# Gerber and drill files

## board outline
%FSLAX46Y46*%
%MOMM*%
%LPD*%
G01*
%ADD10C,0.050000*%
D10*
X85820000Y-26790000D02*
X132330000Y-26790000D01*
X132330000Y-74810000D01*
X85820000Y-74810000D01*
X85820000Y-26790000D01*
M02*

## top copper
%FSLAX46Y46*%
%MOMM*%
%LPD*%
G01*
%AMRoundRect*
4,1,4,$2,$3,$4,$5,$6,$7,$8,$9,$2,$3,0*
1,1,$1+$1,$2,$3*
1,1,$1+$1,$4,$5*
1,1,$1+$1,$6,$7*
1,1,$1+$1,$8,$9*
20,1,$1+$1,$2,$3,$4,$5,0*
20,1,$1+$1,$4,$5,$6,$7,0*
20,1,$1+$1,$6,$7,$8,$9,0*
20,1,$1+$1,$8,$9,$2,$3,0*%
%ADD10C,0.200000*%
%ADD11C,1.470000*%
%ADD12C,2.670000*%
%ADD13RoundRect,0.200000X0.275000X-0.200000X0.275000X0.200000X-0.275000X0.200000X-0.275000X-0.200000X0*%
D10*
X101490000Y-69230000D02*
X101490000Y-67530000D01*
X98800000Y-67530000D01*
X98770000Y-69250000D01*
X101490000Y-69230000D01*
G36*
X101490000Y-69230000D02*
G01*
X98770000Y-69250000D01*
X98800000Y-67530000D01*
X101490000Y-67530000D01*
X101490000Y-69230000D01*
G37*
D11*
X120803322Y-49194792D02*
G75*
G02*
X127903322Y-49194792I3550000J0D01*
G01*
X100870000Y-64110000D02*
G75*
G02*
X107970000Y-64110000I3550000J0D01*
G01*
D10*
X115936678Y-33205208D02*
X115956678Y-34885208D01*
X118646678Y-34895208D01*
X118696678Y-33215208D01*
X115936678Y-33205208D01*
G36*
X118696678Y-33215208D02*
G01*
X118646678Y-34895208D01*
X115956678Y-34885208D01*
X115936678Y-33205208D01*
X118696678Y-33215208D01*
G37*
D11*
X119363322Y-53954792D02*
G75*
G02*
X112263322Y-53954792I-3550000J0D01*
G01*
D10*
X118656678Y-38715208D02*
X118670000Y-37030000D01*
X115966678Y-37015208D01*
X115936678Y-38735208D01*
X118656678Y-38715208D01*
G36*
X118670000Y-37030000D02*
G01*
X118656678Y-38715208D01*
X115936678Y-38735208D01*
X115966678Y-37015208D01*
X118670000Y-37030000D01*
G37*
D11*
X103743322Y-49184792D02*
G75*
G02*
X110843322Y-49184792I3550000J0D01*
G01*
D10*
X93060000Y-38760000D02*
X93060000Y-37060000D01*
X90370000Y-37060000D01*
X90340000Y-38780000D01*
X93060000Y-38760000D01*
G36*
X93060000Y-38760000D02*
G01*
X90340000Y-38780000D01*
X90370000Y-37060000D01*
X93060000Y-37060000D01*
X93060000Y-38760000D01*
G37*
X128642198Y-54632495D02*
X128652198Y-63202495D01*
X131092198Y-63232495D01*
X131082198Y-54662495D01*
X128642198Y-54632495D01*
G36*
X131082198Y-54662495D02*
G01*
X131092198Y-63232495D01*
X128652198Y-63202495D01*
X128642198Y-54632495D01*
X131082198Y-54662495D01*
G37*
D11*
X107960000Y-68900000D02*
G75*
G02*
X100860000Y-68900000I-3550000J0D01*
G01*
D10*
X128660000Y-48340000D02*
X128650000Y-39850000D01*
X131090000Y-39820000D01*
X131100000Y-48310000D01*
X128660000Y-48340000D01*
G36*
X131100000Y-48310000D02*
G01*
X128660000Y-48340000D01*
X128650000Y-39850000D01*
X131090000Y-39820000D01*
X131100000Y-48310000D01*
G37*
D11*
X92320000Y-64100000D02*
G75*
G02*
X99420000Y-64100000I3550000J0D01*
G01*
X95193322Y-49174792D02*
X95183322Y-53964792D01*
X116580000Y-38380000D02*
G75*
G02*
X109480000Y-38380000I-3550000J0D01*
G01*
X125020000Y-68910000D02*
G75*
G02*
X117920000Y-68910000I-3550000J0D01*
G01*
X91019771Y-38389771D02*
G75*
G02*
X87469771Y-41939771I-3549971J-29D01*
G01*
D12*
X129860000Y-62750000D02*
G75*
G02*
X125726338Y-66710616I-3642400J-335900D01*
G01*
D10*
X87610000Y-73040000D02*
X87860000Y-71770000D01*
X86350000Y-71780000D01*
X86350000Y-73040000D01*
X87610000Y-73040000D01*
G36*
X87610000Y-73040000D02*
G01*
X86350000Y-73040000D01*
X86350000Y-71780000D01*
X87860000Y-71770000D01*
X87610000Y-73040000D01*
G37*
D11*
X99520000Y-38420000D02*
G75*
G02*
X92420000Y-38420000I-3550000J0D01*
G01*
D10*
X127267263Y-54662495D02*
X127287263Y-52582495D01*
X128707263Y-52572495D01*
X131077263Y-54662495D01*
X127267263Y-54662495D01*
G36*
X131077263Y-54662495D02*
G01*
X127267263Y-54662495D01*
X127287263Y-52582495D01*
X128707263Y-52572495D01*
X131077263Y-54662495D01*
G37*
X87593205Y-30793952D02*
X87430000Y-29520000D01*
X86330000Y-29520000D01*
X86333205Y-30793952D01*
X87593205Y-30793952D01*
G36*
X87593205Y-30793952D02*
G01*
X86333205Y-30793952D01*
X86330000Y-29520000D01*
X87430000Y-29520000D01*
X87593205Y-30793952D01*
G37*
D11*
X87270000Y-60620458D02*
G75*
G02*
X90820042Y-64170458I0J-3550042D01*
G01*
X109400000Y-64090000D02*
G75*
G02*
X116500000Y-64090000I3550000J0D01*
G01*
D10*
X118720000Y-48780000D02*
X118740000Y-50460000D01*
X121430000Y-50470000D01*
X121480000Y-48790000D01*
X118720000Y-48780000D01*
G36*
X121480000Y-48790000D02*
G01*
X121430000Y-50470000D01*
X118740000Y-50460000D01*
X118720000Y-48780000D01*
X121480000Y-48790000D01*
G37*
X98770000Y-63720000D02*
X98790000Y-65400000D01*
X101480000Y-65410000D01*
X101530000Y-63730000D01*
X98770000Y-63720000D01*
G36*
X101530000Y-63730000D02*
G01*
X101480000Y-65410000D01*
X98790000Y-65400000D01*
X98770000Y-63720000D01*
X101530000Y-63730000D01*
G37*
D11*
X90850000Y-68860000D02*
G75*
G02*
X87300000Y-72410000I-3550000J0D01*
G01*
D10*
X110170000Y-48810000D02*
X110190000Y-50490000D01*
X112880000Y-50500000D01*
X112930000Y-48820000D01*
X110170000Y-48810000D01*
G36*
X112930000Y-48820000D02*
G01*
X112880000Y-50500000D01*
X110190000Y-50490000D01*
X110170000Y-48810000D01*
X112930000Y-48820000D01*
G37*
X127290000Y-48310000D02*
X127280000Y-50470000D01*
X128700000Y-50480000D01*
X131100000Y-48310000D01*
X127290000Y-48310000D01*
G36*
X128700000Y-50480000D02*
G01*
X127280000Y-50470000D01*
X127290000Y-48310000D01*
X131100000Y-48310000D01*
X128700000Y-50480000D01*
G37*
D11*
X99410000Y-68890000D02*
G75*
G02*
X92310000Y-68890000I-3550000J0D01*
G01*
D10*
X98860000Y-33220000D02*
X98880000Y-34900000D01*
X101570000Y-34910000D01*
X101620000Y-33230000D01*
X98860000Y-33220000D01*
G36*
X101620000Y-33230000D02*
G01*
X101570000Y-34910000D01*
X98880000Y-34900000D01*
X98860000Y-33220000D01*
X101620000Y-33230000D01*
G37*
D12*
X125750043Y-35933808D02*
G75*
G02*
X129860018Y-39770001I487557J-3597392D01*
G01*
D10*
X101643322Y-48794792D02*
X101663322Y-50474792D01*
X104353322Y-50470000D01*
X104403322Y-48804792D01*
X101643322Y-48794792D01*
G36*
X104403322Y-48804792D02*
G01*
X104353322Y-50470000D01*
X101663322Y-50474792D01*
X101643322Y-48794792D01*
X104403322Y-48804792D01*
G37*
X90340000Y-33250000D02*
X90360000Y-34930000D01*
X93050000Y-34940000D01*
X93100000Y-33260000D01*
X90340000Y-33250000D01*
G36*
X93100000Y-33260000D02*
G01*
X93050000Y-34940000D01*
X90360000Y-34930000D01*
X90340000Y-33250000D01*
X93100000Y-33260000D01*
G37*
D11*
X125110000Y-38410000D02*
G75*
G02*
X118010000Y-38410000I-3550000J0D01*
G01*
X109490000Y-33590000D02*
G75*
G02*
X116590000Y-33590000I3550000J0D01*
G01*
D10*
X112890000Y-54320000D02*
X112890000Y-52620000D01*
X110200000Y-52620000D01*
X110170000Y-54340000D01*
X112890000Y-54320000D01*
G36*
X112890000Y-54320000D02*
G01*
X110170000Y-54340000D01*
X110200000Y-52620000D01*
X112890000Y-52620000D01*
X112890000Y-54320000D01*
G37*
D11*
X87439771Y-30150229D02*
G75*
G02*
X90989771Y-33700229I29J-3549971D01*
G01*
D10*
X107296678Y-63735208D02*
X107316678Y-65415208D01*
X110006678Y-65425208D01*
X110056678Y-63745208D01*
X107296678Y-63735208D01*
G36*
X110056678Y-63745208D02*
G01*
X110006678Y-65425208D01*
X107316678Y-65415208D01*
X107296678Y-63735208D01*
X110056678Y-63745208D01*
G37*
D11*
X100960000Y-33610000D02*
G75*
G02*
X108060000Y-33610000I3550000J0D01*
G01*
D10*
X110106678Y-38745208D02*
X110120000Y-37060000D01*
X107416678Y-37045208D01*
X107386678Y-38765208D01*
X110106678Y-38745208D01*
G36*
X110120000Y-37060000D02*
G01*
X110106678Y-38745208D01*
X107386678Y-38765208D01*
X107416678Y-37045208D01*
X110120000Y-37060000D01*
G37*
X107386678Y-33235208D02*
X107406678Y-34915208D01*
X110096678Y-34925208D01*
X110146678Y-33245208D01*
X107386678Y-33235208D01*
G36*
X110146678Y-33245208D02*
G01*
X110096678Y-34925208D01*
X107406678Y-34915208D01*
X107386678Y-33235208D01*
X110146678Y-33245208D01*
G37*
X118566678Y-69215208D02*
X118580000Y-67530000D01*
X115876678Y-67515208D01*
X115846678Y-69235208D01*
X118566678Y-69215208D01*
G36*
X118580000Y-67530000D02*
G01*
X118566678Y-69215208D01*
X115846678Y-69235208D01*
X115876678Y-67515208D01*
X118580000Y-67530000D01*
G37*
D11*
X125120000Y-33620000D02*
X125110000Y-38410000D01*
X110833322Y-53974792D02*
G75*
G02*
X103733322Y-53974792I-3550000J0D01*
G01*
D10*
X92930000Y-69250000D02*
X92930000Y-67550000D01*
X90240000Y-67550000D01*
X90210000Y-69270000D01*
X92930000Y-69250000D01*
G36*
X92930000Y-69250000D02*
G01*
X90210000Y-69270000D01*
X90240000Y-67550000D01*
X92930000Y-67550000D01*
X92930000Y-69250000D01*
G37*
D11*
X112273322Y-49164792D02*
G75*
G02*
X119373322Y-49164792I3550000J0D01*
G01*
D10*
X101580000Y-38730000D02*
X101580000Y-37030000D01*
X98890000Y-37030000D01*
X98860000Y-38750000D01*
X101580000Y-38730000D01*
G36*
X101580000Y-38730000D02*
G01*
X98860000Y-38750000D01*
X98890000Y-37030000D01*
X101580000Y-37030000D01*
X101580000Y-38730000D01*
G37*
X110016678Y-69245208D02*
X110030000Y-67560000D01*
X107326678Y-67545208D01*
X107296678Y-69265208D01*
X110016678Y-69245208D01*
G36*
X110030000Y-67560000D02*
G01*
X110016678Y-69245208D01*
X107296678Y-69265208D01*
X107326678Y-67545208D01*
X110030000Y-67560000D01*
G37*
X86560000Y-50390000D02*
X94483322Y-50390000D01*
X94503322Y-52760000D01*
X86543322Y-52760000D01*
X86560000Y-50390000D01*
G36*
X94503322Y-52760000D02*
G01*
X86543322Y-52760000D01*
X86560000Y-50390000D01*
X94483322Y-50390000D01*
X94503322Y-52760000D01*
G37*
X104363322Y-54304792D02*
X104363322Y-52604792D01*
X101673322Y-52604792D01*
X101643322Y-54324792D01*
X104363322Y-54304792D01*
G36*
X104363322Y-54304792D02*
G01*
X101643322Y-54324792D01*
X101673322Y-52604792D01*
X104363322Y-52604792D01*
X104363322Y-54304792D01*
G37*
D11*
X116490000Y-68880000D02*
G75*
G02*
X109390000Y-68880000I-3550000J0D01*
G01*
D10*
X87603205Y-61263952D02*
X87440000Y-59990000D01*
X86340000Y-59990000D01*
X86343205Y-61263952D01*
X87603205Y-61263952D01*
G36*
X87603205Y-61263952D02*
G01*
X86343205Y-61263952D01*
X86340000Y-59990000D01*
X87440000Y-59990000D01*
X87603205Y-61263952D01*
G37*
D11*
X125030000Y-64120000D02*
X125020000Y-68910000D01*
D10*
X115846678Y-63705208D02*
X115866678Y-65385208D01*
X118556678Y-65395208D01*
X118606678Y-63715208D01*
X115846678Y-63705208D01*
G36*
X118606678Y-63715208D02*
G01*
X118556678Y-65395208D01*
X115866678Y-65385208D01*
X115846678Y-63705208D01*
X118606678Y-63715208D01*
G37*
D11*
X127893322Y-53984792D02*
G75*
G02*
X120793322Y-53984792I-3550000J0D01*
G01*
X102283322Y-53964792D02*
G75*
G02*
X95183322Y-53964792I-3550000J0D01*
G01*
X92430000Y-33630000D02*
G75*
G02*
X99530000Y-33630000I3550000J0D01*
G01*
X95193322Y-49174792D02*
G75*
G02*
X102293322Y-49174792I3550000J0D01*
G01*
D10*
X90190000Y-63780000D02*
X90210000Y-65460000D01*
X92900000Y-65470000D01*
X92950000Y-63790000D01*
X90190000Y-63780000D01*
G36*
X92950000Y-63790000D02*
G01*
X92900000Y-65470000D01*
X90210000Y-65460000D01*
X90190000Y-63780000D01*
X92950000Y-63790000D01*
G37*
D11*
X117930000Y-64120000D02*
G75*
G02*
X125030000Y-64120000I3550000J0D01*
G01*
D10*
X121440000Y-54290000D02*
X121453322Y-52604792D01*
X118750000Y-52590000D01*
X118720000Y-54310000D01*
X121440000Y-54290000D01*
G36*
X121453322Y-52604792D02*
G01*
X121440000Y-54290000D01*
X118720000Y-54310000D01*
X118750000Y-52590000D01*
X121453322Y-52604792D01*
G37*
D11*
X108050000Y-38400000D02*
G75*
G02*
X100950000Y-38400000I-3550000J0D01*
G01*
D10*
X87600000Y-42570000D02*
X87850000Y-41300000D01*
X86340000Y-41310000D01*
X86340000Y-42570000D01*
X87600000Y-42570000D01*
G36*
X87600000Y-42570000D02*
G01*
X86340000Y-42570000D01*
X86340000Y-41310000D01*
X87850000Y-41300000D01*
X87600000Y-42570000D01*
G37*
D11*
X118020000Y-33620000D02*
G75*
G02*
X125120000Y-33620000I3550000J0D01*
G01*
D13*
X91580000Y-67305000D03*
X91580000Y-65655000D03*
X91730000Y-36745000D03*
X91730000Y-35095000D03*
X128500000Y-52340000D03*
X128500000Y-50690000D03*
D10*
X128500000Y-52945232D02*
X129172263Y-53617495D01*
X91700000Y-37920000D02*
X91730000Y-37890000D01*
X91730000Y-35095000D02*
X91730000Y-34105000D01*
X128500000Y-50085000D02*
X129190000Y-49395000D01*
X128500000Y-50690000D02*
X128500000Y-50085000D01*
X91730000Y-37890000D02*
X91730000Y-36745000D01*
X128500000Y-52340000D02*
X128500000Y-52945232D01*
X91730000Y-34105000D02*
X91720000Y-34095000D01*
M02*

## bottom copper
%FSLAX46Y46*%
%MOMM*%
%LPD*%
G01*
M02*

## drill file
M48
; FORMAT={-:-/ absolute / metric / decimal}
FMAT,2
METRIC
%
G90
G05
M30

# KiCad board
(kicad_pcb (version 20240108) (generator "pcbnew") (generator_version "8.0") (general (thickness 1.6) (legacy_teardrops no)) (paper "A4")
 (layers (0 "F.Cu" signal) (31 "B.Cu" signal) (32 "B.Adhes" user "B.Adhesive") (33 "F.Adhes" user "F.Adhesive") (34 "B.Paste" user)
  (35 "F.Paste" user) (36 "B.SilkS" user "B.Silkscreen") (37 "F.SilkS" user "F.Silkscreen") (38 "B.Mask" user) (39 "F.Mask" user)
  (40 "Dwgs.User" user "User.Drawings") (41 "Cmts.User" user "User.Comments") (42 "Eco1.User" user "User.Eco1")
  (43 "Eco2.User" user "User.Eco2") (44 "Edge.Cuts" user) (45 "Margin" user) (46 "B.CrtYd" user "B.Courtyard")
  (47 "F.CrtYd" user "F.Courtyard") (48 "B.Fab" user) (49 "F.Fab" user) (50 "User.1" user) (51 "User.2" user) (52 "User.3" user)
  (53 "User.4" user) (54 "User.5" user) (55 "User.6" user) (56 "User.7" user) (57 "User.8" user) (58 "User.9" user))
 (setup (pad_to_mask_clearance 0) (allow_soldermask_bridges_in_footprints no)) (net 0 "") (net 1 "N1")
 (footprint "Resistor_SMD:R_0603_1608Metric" (layer "F.Cu") (at 91.58 66.48 90)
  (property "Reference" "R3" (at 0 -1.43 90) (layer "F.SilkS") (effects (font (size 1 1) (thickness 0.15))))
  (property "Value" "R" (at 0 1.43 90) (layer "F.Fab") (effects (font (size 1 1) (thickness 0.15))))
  (pad "1" smd roundrect (at -0.825 0 90) (size 0.8 0.95) (layers "F.Cu" "F.Paste" "F.Mask") (roundrect_rratio 0.25) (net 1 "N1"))
  (pad "2" smd roundrect (at 0.825 0 90) (size 0.8 0.95) (layers "F.Cu" "F.Paste" "F.Mask") (roundrect_rratio 0.25) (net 1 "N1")))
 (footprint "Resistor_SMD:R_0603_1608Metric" (layer "F.Cu") (at 91.73 35.92 90)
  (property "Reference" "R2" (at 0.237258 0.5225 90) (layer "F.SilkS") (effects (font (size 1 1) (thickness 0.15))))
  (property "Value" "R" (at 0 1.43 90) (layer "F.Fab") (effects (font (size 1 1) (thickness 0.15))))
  (pad "1" smd roundrect (at -0.825 0 90) (size 0.8 0.95) (layers "F.Cu" "F.Paste" "F.Mask") (roundrect_rratio 0.25) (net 1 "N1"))
  (pad "2" smd roundrect (at 0.825 0 90) (size 0.8 0.95) (layers "F.Cu" "F.Paste" "F.Mask") (roundrect_rratio 0.25) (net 1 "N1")))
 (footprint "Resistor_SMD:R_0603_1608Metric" (layer "F.Cu") (at 128.5 51.515 90)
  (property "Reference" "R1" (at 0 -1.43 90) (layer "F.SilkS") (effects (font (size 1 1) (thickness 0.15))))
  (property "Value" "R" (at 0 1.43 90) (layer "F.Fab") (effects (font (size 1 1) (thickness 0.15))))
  (pad "1" smd roundrect (at -0.825 0 90) (size 0.8 0.95) (layers "F.Cu" "F.Paste" "F.Mask") (roundrect_rratio 0.25) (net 1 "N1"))
  (pad "2" smd roundrect (at 0.825 0 90) (size 0.8 0.95) (layers "F.Cu" "F.Paste" "F.Mask") (roundrect_rratio 0.25) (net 1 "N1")))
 (gr_poly
  (pts (xy 101.49 69.23) (xy 101.49 67.53) (xy 98.8 67.53) (xy 98.77 69.25)) (stroke (width 0.2) (type solid)) (fill solid) (layer "F.Cu")
  (net 1))
 (gr_arc (start 120.803322 49.194792) (mid 124.353322 45.644792) (end 127.903322 49.194792) (stroke (width 1.47) (type default))
  (layer "F.Cu") (net 1))
 (gr_arc (start 100.87 64.11) (mid 104.42 60.56) (end 107.97 64.11) (stroke (width 1.47) (type default)) (layer "F.Cu") (net 1))
 (gr_poly
  (pts (xy 115.936678 33.205208) (xy 115.956678 34.885208) (xy 118.646678 34.895208) (xy 118.696678 33.215208))
  (stroke (width 0.2) (type solid)) (fill solid) (layer "F.Cu") (net 1))
 (gr_arc (start 119.363322 53.954792) (mid 115.813322 57.504792) (end 112.263322 53.954792) (stroke (width 1.47) (type default))
  (layer "F.Cu") (net 1))
 (gr_poly
  (pts (xy 118.656678 38.715208) (xy 118.67 37.03) (xy 115.966678 37.015208) (xy 115.936678 38.735208)) (stroke (width 0.2) (type solid))
  (fill solid) (layer "F.Cu") (net 1))
 (gr_arc (start 103.743322 49.184792) (mid 107.293322 45.634792) (end 110.843322 49.184792) (stroke (width 1.47) (type default))
  (layer "F.Cu") (net 1))
 (gr_poly
  (pts (xy 93.06 38.76) (xy 93.06 37.06) (xy 90.37 37.06) (xy 90.34 38.78)) (stroke (width 0.2) (type solid)) (fill solid) (layer "F.Cu")
  (net 1))
 (gr_poly
  (pts (xy 128.642198 54.632495) (xy 128.652198 63.202495) (xy 131.092198 63.232495) (xy 131.082198 54.662495))
  (stroke (width 0.2) (type solid)) (fill solid) (layer "F.Cu") (net 1))
 (gr_arc (start 107.96 68.9) (mid 104.41 72.45) (end 100.86 68.9) (stroke (width 1.47) (type default)) (layer "F.Cu") (net 1))
 (gr_poly
  (pts (xy 128.66 48.34) (xy 128.65 39.85) (xy 131.09 39.82) (xy 131.1 48.31)) (stroke (width 0.2) (type solid)) (fill solid) (layer "F.Cu")
  (net 1))
 (gr_arc (start 92.32 64.1) (mid 95.87 60.55) (end 99.42 64.1) (stroke (width 1.47) (type default)) (layer "F.Cu") (net 1))
 (gr_line (start 95.193322 49.174792) (end 95.183322 53.964792) (stroke (width 1.47) (type default)) (layer "F.Cu") (net 1))
 (gr_arc (start 116.58 38.38) (mid 113.03 41.93) (end 109.48 38.38) (stroke (width 1.47) (type default)) (layer "F.Cu") (net 1))
 (gr_arc (start 125.02 68.91) (mid 121.47 72.46) (end 117.92 68.91) (stroke (width 1.47) (type default)) (layer "F.Cu") (net 1))
 (gr_arc (start 91.019771 38.389771) (mid 89.98 40.9) (end 87.469771 41.939771) (stroke (width 1.47) (type default)) (layer "F.Cu") (net 1))
 (gr_arc (start 129.86 62.75) (mid 128.748221 65.727091) (end 125.726337 66.710626) (stroke (width 2.67) (type default)) (layer "F.Cu")
  (net 1))
 (gr_poly
  (pts (xy 87.61 73.04) (xy 87.86 71.77) (xy 86.35 71.78) (xy 86.35 73.04)) (stroke (width 0.2) (type solid)) (fill solid) (layer "F.Cu")
  (net 1))
 (gr_arc (start 99.52 38.42) (mid 95.97 41.97) (end 92.42 38.42) (stroke (width 1.47) (type default)) (layer "F.Cu") (net 1))
 (gr_poly
  (pts (xy 127.267263 54.662495) (xy 127.287263 52.582495) (xy 128.707263 52.572495) (xy 131.077263 54.662495))
  (stroke (width 0.2) (type solid)) (fill solid) (layer "F.Cu") (net 1))
 (gr_poly
  (pts (xy 87.593205 30.793952) (xy 87.43 29.52) (xy 86.33 29.52) (xy 86.333205 30.793952)) (stroke (width 0.2) (type solid)) (fill solid)
  (layer "F.Cu") (net 1))
 (gr_arc (start 87.27 60.620458) (mid 89.780229 61.660229) (end 90.82 64.170458) (stroke (width 1.47) (type default)) (layer "F.Cu") (net 1))
 (gr_arc (start 109.4 64.09) (mid 112.95 60.54) (end 116.5 64.09) (stroke (width 1.47) (type default)) (layer "F.Cu") (net 1))
 (gr_poly
  (pts (xy 118.72 48.78) (xy 118.74 50.46) (xy 121.43 50.47) (xy 121.48 48.79)) (stroke (width 0.2) (type solid)) (fill solid)
  (layer "F.Cu") (net 1))
 (gr_poly
  (pts (xy 98.77 63.72) (xy 98.79 65.4) (xy 101.48 65.41) (xy 101.53 63.73)) (stroke (width 0.2) (type solid)) (fill solid) (layer "F.Cu")
  (net 1))
 (gr_arc (start 90.85 68.86) (mid 89.810229 71.370229) (end 87.3 72.41) (stroke (width 1.47) (type default)) (layer "F.Cu") (net 1))
 (gr_poly
  (pts (xy 110.17 48.81) (xy 110.19 50.49) (xy 112.88 50.5) (xy 112.93 48.82)) (stroke (width 0.2) (type solid)) (fill solid) (layer "F.Cu")
  (net 1))
 (gr_poly
  (pts (xy 127.29 48.31) (xy 127.28 50.47) (xy 128.7 50.48) (xy 131.1 48.31)) (stroke (width 0.2) (type solid)) (fill solid) (layer "F.Cu")
  (net 1))
 (gr_arc (start 99.41 68.89) (mid 95.86 72.44) (end 92.31 68.89) (stroke (width 1.47) (type default)) (layer "F.Cu") (net 1))
 (gr_poly
  (pts (xy 98.86 33.22) (xy 98.88 34.9) (xy 101.57 34.91) (xy 101.62 33.23)) (stroke (width 0.2) (type solid)) (fill solid) (layer "F.Cu")
  (net 1))
 (gr_arc (start 125.750043 35.933808) (mid 128.714673 36.877337) (end 129.86 39.77) (stroke (width 2.67) (type default)) (layer "F.Cu")
  (net 1))
 (gr_poly
  (pts (xy 101.643322 48.794792) (xy 101.663322 50.474792) (xy 104.353322 50.47) (xy 104.403322 48.804792))
  (stroke (width 0.2) (type solid)) (fill solid) (layer "F.Cu") (net 1))
 (gr_poly
  (pts (xy 90.34 33.25) (xy 90.36 34.93) (xy 93.05 34.94) (xy 93.1 33.26)) (stroke (width 0.2) (type solid)) (fill solid) (layer "F.Cu")
  (net 1))
 (gr_arc (start 125.11 38.41) (mid 121.56 41.96) (end 118.01 38.41) (stroke (width 1.47) (type default)) (layer "F.Cu") (net 1))
 (gr_arc (start 109.49 33.59) (mid 113.04 30.04) (end 116.59 33.59) (stroke (width 1.47) (type default)) (layer "F.Cu") (net 1))
 (gr_poly
  (pts (xy 112.89 54.32) (xy 112.89 52.62) (xy 110.2 52.62) (xy 110.17 54.34)) (stroke (width 0.2) (type solid)) (fill solid) (layer "F.Cu")
  (net 1))
 (gr_arc (start 87.439771 30.150229) (mid 89.95 31.19) (end 90.989771 33.700229) (stroke (width 1.47) (type default)) (layer "F.Cu") (net 1))
 (gr_poly
  (pts (xy 107.296678 63.735208) (xy 107.316678 65.415208) (xy 110.006678 65.425208) (xy 110.056678 63.745208))
  (stroke (width 0.2) (type solid)) (fill solid) (layer "F.Cu") (net 1))
 (gr_arc (start 100.96 33.61) (mid 104.51 30.06) (end 108.06 33.61) (stroke (width 1.47) (type default)) (layer "F.Cu") (net 1))
 (gr_poly
  (pts (xy 110.106678 38.745208) (xy 110.12 37.06) (xy 107.416678 37.045208) (xy 107.386678 38.765208)) (stroke (width 0.2) (type solid))
  (fill solid) (layer "F.Cu") (net 1))
 (gr_poly
  (pts (xy 107.386678 33.235208) (xy 107.406678 34.915208) (xy 110.096678 34.925208) (xy 110.146678 33.245208))
  (stroke (width 0.2) (type solid)) (fill solid) (layer "F.Cu") (net 1))
 (gr_poly
  (pts (xy 118.566678 69.215208) (xy 118.58 67.53) (xy 115.876678 67.515208) (xy 115.846678 69.235208)) (stroke (width 0.2) (type solid))
  (fill solid) (layer "F.Cu") (net 1))
 (gr_line (start 125.12 33.62) (end 125.11 38.41) (stroke (width 1.47) (type default)) (layer "F.Cu") (net 1))
 (gr_arc (start 110.833322 53.974792) (mid 107.283322 57.524792) (end 103.733322 53.974792) (stroke (width 1.47) (type default))
  (layer "F.Cu") (net 1))
 (gr_poly
  (pts (xy 92.93 69.25) (xy 92.93 67.55) (xy 90.24 67.55) (xy 90.21 69.27)) (stroke (width 0.2) (type solid)) (fill solid) (layer "F.Cu")
  (net 1))
 (gr_arc (start 112.273322 49.164792) (mid 115.823322 45.614792) (end 119.373322 49.164792) (stroke (width 1.47) (type default))
  (layer "F.Cu") (net 1))
 (gr_poly
  (pts (xy 101.58 38.73) (xy 101.58 37.03) (xy 98.89 37.03) (xy 98.86 38.75)) (stroke (width 0.2) (type solid)) (fill solid) (layer "F.Cu")
  (net 1))
 (gr_poly
  (pts (xy 110.016678 69.245208) (xy 110.03 67.56) (xy 107.326678 67.545208) (xy 107.296678 69.265208)) (stroke (width 0.2) (type solid))
  (fill solid) (layer "F.Cu") (net 1))
 (gr_poly
  (pts (xy 86.56 50.39) (xy 94.483322 50.39) (xy 94.503322 52.76) (xy 86.543322 52.76)) (stroke (width 0.2) (type solid)) (fill solid)
  (layer "F.Cu") (net 1))
 (gr_poly
  (pts (xy 104.363322 54.304792) (xy 104.363322 52.604792) (xy 101.673322 52.604792) (xy 101.643322 54.324792))
  (stroke (width 0.2) (type solid)) (fill solid) (layer "F.Cu") (net 1))
 (gr_arc (start 116.49 68.88) (mid 112.94 72.43) (end 109.39 68.88) (stroke (width 1.47) (type default)) (layer "F.Cu") (net 1))
 (gr_poly
  (pts (xy 87.603205 61.263952) (xy 87.44 59.99) (xy 86.34 59.99) (xy 86.343205 61.263952)) (stroke (width 0.2) (type solid)) (fill solid)
  (layer "F.Cu") (net 1))
 (gr_line (start 125.03 64.12) (end 125.02 68.91) (stroke (width 1.47) (type default)) (layer "F.Cu") (net 1))
 (gr_poly
  (pts (xy 115.846678 63.705208) (xy 115.866678 65.385208) (xy 118.556678 65.395208) (xy 118.606678 63.715208))
  (stroke (width 0.2) (type solid)) (fill solid) (layer "F.Cu") (net 1))
 (gr_arc (start 127.893322 53.984792) (mid 124.343322 57.534792) (end 120.793322 53.984792) (stroke (width 1.47) (type default))
  (layer "F.Cu") (net 1))
 (gr_arc (start 102.283322 53.964792) (mid 98.733322 57.514792) (end 95.183322 53.964792) (stroke (width 1.47) (type default))
  (layer "F.Cu") (net 1))
 (gr_arc (start 92.43 33.63) (mid 95.98 30.08) (end 99.53 33.63) (stroke (width 1.47) (type default)) (layer "F.Cu") (net 1))
 (gr_arc (start 95.193322 49.174792) (mid 98.743322 45.624792) (end 102.293322 49.174792) (stroke (width 1.47) (type default))
  (layer "F.Cu") (net 1))
 (gr_poly
  (pts (xy 90.19 63.78) (xy 90.21 65.46) (xy 92.9 65.47) (xy 92.95 63.79)) (stroke (width 0.2) (type solid)) (fill solid) (layer "F.Cu")
  (net 1))
 (gr_arc (start 117.93 64.12) (mid 121.48 60.57) (end 125.03 64.12) (stroke (width 1.47) (type default)) (layer "F.Cu") (net 1))
 (gr_poly
  (pts (xy 121.44 54.29) (xy 121.453322 52.604792) (xy 118.75 52.59) (xy 118.72 54.31)) (stroke (width 0.2) (type solid)) (fill solid)
  (layer "F.Cu") (net 1))
 (gr_arc (start 108.05 38.4) (mid 104.5 41.95) (end 100.95 38.4) (stroke (width 1.47) (type default)) (layer "F.Cu") (net 1))
 (gr_poly
  (pts (xy 87.6 42.57) (xy 87.85 41.3) (xy 86.34 41.31) (xy 86.34 42.57)) (stroke (width 0.2) (type solid)) (fill solid) (layer "F.Cu")
  (net 1))
 (gr_arc (start 118.02 33.62) (mid 121.57 30.07) (end 125.12 33.62) (stroke (width 1.47) (type default)) (layer "F.Cu") (net 1))
 (gr_rect (start 85.82 26.79) (end 132.33 74.81) (stroke (width 0.05) (type default)) (fill none) (layer "Edge.Cuts"))
 (segment (start 128.5 52.945232) (end 129.172263 53.617495) (width 0.2) (layer "F.Cu") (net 1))
 (segment (start 91.7 37.92) (end 91.73 37.89) (width 0.2) (layer "F.Cu") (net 1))
 (segment (start 91.73 35.095) (end 91.73 34.105) (width 0.2) (layer "F.Cu") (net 1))
 (segment (start 128.5 50.085) (end 129.19 49.395) (width 0.2) (layer "F.Cu") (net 1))
 (segment (start 128.5 50.69) (end 128.5 50.085) (width 0.2) (layer "F.Cu") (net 1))
 (segment (start 91.73 37.89) (end 91.73 36.745) (width 0.2) (layer "F.Cu") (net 1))
 (segment (start 128.5 52.34) (end 128.5 52.945232) (width 0.2) (layer "F.Cu") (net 1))
 (segment (start 91.73 34.105) (end 91.72 34.095) (width 0.2) (layer "F.Cu") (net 1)))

